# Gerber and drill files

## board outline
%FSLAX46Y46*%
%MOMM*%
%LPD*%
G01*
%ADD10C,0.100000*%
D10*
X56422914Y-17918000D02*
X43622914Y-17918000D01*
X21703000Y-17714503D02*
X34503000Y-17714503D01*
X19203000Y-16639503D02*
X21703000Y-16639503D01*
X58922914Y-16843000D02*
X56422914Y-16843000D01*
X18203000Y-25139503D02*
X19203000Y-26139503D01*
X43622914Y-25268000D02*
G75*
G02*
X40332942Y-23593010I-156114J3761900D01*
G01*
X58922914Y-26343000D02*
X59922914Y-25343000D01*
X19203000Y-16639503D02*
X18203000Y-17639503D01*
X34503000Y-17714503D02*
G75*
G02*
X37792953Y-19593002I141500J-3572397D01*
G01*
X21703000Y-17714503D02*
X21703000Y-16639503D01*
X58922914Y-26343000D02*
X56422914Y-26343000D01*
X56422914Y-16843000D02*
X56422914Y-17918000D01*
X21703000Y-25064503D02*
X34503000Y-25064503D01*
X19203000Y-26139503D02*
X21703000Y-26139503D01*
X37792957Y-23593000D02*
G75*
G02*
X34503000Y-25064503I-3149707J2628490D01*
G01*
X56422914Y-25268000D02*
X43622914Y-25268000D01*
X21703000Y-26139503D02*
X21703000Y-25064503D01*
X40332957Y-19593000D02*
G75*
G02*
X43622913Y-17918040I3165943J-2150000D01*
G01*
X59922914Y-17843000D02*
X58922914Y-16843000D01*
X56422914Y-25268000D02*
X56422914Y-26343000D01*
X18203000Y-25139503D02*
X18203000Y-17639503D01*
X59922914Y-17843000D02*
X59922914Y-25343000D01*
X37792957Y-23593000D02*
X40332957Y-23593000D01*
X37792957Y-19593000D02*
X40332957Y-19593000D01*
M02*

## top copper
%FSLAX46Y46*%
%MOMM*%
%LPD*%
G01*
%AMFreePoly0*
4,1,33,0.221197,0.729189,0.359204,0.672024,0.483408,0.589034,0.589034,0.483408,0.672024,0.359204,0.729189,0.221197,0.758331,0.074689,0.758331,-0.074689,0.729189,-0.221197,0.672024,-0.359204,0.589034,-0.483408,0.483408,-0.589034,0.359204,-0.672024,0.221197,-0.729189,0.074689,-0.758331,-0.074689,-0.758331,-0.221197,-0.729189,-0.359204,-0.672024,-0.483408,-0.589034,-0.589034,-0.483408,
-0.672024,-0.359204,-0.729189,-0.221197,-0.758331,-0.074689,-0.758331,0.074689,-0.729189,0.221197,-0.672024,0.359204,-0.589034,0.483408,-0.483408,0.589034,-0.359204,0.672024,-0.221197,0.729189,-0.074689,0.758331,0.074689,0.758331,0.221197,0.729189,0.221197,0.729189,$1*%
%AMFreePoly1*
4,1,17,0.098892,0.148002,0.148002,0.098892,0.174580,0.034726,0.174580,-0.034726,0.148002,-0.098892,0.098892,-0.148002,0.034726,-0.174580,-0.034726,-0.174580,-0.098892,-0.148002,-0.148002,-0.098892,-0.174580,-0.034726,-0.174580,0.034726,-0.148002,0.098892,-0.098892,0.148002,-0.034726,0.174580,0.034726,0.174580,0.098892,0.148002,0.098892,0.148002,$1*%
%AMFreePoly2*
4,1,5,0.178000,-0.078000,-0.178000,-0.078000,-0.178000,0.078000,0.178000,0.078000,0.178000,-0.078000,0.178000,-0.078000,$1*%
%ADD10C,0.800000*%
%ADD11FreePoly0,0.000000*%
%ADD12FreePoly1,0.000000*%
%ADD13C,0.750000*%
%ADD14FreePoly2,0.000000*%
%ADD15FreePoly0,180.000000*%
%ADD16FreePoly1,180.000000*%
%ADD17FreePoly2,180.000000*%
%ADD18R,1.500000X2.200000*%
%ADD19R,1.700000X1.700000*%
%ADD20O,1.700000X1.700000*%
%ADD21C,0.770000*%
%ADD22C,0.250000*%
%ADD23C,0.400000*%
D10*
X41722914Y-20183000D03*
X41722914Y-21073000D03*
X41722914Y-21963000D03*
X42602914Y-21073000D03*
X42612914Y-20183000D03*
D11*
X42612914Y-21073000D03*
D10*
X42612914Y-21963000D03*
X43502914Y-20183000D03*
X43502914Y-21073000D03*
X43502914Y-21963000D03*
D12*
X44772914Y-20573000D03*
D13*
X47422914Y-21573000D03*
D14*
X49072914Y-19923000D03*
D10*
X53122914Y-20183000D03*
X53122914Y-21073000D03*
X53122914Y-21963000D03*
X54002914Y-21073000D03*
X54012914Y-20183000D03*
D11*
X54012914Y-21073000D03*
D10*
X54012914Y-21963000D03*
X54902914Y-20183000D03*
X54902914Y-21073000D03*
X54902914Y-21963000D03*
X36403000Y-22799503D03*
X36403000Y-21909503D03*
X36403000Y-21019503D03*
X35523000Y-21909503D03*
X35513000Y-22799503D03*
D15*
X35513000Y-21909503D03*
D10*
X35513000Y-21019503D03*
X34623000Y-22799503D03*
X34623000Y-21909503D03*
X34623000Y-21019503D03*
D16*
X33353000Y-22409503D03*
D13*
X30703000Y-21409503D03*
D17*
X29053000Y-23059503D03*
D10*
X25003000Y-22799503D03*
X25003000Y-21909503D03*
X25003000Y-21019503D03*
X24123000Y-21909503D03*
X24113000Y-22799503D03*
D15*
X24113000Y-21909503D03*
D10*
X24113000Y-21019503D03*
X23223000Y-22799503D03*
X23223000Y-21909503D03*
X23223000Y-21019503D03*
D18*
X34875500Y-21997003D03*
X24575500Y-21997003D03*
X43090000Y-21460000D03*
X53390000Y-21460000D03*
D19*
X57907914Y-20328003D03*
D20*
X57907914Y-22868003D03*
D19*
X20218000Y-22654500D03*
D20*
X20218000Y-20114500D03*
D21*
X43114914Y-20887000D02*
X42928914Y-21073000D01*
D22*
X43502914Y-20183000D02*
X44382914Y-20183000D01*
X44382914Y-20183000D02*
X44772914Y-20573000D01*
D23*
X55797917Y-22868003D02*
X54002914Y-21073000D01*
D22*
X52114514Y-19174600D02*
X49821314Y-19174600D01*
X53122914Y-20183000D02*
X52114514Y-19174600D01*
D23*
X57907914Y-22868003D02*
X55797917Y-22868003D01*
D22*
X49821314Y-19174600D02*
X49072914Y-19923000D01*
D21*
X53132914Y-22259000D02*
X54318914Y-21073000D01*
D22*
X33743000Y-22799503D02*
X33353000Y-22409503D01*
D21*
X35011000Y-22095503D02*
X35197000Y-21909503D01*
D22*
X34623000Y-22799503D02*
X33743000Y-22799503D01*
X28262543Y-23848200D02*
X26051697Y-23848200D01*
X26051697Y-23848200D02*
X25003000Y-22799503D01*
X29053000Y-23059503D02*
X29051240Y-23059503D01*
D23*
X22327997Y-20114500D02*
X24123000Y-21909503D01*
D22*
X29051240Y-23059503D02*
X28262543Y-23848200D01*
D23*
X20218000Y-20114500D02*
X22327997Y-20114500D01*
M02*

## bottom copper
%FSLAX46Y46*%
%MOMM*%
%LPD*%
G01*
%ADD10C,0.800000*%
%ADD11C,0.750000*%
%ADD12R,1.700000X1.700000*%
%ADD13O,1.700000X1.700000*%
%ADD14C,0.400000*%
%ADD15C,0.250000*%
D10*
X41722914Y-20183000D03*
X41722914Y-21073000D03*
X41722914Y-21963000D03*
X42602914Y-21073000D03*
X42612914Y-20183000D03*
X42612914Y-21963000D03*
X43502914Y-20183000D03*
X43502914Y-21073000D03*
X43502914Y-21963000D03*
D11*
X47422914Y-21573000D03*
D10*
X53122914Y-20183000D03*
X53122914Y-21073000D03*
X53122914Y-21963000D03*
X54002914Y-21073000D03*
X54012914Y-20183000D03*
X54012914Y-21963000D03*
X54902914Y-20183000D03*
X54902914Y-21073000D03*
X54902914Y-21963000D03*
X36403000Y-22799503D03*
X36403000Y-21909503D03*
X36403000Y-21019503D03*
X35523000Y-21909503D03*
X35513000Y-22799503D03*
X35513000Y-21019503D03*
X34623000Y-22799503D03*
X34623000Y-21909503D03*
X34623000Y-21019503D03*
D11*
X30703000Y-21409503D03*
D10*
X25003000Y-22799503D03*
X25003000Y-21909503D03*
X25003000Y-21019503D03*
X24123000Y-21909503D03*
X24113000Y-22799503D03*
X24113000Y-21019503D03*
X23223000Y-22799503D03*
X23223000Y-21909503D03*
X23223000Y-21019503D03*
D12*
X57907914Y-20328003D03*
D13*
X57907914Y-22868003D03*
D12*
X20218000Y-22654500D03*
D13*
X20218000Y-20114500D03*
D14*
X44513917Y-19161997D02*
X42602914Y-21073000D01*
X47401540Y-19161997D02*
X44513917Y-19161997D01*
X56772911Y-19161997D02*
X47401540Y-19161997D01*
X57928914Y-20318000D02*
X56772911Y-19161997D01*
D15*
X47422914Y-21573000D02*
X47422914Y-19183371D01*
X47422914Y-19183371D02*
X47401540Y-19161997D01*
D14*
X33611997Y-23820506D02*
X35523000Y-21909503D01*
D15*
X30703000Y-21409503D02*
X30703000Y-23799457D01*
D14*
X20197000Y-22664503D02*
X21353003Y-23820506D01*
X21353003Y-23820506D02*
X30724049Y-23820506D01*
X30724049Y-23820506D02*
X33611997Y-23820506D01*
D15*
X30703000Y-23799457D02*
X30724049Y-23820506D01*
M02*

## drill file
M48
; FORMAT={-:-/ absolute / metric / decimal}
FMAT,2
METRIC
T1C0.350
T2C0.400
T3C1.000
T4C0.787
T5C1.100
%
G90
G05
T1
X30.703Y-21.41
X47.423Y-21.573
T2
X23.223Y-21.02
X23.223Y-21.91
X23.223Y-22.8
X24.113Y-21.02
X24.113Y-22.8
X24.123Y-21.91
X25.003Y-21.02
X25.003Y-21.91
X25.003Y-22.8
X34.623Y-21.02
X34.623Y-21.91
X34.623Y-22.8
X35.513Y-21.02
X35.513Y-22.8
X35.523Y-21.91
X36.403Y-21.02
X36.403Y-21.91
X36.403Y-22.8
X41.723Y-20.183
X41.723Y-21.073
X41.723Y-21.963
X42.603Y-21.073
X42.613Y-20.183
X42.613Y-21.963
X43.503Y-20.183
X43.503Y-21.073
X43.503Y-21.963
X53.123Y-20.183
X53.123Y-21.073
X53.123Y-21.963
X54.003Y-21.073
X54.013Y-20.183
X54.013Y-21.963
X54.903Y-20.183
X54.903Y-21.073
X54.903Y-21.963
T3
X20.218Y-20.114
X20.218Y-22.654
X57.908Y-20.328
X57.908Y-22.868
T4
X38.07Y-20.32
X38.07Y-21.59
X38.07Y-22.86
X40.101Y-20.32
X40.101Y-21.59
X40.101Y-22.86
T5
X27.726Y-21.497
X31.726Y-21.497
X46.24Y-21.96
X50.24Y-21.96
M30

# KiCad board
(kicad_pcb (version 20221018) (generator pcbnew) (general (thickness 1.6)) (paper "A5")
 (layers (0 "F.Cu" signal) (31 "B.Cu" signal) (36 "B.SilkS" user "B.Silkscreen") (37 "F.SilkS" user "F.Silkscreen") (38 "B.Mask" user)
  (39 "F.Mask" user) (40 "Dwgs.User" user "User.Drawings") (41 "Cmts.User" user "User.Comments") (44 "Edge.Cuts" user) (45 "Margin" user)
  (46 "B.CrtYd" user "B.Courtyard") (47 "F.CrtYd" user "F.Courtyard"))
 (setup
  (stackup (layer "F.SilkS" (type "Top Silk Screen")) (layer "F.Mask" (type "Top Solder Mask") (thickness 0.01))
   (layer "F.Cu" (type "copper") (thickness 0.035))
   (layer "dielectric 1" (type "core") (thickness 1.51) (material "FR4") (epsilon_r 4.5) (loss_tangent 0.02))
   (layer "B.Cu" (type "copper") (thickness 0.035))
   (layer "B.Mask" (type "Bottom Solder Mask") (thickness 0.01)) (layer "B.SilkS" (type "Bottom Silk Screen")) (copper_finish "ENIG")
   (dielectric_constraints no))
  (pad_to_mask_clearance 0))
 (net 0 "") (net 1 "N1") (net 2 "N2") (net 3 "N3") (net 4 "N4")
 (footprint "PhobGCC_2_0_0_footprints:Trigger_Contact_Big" (layer "F.Cu") (at 47.422914 21.573)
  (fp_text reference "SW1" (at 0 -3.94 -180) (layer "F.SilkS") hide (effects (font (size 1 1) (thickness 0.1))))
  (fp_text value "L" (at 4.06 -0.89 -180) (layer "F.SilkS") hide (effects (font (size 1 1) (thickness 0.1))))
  (pad "1" thru_hole circle (at -5.7 -1.39) (size 0.8 0.8) (drill 0.4) (layers "*.Cu" "*.Mask") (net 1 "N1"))
  (pad "1" thru_hole circle (at -5.7 -0.5) (size 0.8 0.8) (drill 0.4) (layers "*.Cu" "*.Mask") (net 1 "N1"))
  (pad "1" thru_hole circle (at -5.7 0.39) (size 0.8 0.8) (drill 0.4) (layers "*.Cu" "*.Mask") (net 1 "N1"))
  (pad "1" thru_hole circle (at -4.82 -0.5) (size 0.8 0.8) (drill 0.4) (layers "*.Cu" "*.Mask") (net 1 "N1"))
  (pad "1" thru_hole circle (at -4.81 -1.39) (size 0.8 0.8) (drill 0.4) (layers "*.Cu" "*.Mask") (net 1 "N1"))
  (pad "1" smd custom (at -4.81 -0.5) (size 1.524 1.524) (layers "F.Cu" "F.Paste" "F.Mask") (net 1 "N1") (thermal_bridge_angle 45)
   (options (clearance outline) (anchor circle)) (primitives))
  (pad "1" thru_hole circle (at -4.81 0.39) (size 0.8 0.8) (drill 0.4) (layers "*.Cu" "*.Mask") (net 1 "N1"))
  (pad "1" thru_hole circle (at -3.92 -1.39) (size 0.8 0.8) (drill 0.4) (layers "*.Cu" "*.Mask") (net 1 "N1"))
  (pad "1" thru_hole circle (at -3.92 -0.5) (size 0.8 0.8) (drill 0.4) (layers "*.Cu" "*.Mask") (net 1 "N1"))
  (pad "1" thru_hole circle (at -3.92 0.39) (size 0.8 0.8) (drill 0.4) (layers "*.Cu" "*.Mask") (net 1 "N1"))
  (pad "1" smd custom (at -2.65 -1) (size 0.356 0.356) (layers "F.Cu" "F.Paste" "F.Mask") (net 1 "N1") (thermal_bridge_angle 45)
   (options (clearance outline) (anchor circle)) (primitives))
  (pad "1" thru_hole circle (at 0 0) (size 0.75 0.75) (drill 0.35) (layers "*.Cu" "*.Mask") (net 1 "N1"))
  (pad "2" smd custom (at 1.65 -1.65) (size 0.356 0.156) (layers "F.Cu" "F.Paste" "F.Mask") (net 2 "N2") (thermal_bridge_angle 45)
   (options (clearance outline) (anchor rect)) (primitives))
  (pad "2" thru_hole circle (at 5.7 -1.39) (size 0.8 0.8) (drill 0.4) (layers "*.Cu" "*.Mask") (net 2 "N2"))
  (pad "2" thru_hole circle (at 5.7 -0.5) (size 0.8 0.8) (drill 0.4) (layers "*.Cu" "*.Mask") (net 2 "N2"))
  (pad "2" thru_hole circle (at 5.7 0.39) (size 0.8 0.8) (drill 0.4) (layers "*.Cu" "*.Mask") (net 2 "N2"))
  (pad "2" thru_hole circle (at 6.58 -0.5) (size 0.8 0.8) (drill 0.4) (layers "*.Cu" "*.Mask") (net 2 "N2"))
  (pad "2" thru_hole circle (at 6.59 -1.39) (size 0.8 0.8) (drill 0.4) (layers "*.Cu" "*.Mask") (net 2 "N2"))
  (pad "2" smd custom (at 6.59 -0.5) (size 1.524 1.524) (layers "F.Cu" "F.Paste" "F.Mask") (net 2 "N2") (thermal_bridge_angle 45)
   (options (clearance outline) (anchor circle)) (primitives))
  (pad "2" thru_hole circle (at 6.59 0.39) (size 0.8 0.8) (drill 0.4) (layers "*.Cu" "*.Mask") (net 2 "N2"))
  (pad "2" thru_hole circle (at 7.48 -1.39) (size 0.8 0.8) (drill 0.4) (layers "*.Cu" "*.Mask") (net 2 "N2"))
  (pad "2" thru_hole circle (at 7.48 -0.5) (size 0.8 0.8) (drill 0.4) (layers "*.Cu" "*.Mask") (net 2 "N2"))
  (pad "2" thru_hole circle (at 7.48 0.39) (size 0.8 0.8) (drill 0.4) (layers "*.Cu" "*.Mask") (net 2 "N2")))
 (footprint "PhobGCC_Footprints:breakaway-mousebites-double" (layer "F.Cu") (at 40.33085 21.36 90)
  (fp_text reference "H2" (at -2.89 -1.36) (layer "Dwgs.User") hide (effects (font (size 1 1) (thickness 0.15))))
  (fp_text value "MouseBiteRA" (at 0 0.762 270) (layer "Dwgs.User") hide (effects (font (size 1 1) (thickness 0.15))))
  (fp_line (start -2.233 -2.537893) (end -2.233 0.002107) (stroke (width 0.1) (type solid)) (layer "Edge.Cuts"))
  (fp_line (start 1.767 -2.537893) (end 1.767 0.002107) (stroke (width 0.1) (type solid)) (layer "Edge.Cuts"))
  (pad "" np_thru_hole circle (at -1.5 -2.26085 270) (size 0.7874 0.7874) (drill 0.7874) (layers "*.Cu" "*.Mask"))
  (pad "" np_thru_hole circle (at -1.5 -0.23 90) (size 0.7874 0.7874) (drill 0.7874) (layers "*.Cu" "*.Mask"))
  (pad "" np_thru_hole circle (at -0.23 -2.26085 270) (size 0.7874 0.7874) (drill 0.7874) (layers "*.Cu" "*.Mask"))
  (pad "" np_thru_hole circle (at -0.23 -0.23 90) (size 0.7874 0.7874) (drill 0.7874) (layers "*.Cu" "*.Mask"))
  (pad "" np_thru_hole circle (at 1.04 -2.26085 270) (size 0.7874 0.7874) (drill 0.7874) (layers "*.Cu" "*.Mask"))
  (pad "" np_thru_hole circle (at 1.04 -0.23 90) (size 0.7874 0.7874) (drill 0.7874) (layers "*.Cu" "*.Mask")))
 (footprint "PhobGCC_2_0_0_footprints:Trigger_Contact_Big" (layer "F.Cu") (at 30.703 21.409503 180)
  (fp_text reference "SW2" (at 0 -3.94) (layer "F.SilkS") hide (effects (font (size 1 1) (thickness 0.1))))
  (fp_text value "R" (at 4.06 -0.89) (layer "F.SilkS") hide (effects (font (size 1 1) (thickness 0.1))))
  (pad "1" thru_hole circle (at -5.7 -1.39 180) (size 0.8 0.8) (drill 0.4) (layers "*.Cu" "*.Mask") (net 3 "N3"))
  (pad "1" thru_hole circle (at -5.7 -0.5 180) (size 0.8 0.8) (drill 0.4) (layers "*.Cu" "*.Mask") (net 3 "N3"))
  (pad "1" thru_hole circle (at -5.7 0.39 180) (size 0.8 0.8) (drill 0.4) (layers "*.Cu" "*.Mask") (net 3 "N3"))
  (pad "1" thru_hole circle (at -4.82 -0.5 180) (size 0.8 0.8) (drill 0.4) (layers "*.Cu" "*.Mask") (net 3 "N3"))
  (pad "1" thru_hole circle (at -4.81 -1.39 180) (size 0.8 0.8) (drill 0.4) (layers "*.Cu" "*.Mask") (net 3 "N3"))
  (pad "1" smd custom (at -4.81 -0.5 180) (size 1.524 1.524) (layers "F.Cu" "F.Paste" "F.Mask") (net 3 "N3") (thermal_bridge_angle 45)
   (options (clearance outline) (anchor circle)) (primitives))
  (pad "1" thru_hole circle (at -4.81 0.39 180) (size 0.8 0.8) (drill 0.4) (layers "*.Cu" "*.Mask") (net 3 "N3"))
  (pad "1" thru_hole circle (at -3.92 -1.39 180) (size 0.8 0.8) (drill 0.4) (layers "*.Cu" "*.Mask") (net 3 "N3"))
  (pad "1" thru_hole circle (at -3.92 -0.5 180) (size 0.8 0.8) (drill 0.4) (layers "*.Cu" "*.Mask") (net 3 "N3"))
  (pad "1" thru_hole circle (at -3.92 0.39 180) (size 0.8 0.8) (drill 0.4) (layers "*.Cu" "*.Mask") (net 3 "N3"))
  (pad "1" smd custom (at -2.65 -1 180) (size 0.356 0.356) (layers "F.Cu" "F.Paste" "F.Mask") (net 3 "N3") (thermal_bridge_angle 45)
   (options (clearance outline) (anchor circle)) (primitives))
  (pad "1" thru_hole circle (at 0 0 180) (size 0.75 0.75) (drill 0.35) (layers "*.Cu" "*.Mask") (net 3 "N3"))
  (pad "2" smd custom (at 1.65 -1.65 180) (size 0.356 0.156) (layers "F.Cu" "F.Paste" "F.Mask") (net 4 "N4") (thermal_bridge_angle 45)
   (options (clearance outline) (anchor rect)) (primitives))
  (pad "2" thru_hole circle (at 5.7 -1.39 180) (size 0.8 0.8) (drill 0.4) (layers "*.Cu" "*.Mask") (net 4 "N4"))
  (pad "2" thru_hole circle (at 5.7 -0.5 180) (size 0.8 0.8) (drill 0.4) (layers "*.Cu" "*.Mask") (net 4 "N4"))
  (pad "2" thru_hole circle (at 5.7 0.39 180) (size 0.8 0.8) (drill 0.4) (layers "*.Cu" "*.Mask") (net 4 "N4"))
  (pad "2" thru_hole circle (at 6.58 -0.5 180) (size 0.8 0.8) (drill 0.4) (layers "*.Cu" "*.Mask") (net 4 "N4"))
  (pad "2" thru_hole circle (at 6.59 -1.39 180) (size 0.8 0.8) (drill 0.4) (layers "*.Cu" "*.Mask") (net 4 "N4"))
  (pad "2" smd custom (at 6.59 -0.5 180) (size 1.524 1.524) (layers "F.Cu" "F.Paste" "F.Mask") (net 4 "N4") (thermal_bridge_angle 45)
   (options (clearance outline) (anchor circle)) (primitives))
  (pad "2" thru_hole circle (at 6.59 0.39 180) (size 0.8 0.8) (drill 0.4) (layers "*.Cu" "*.Mask") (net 4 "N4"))
  (pad "2" thru_hole circle (at 7.48 -1.39 180) (size 0.8 0.8) (drill 0.4) (layers "*.Cu" "*.Mask") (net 4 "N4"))
  (pad "2" thru_hole circle (at 7.48 -0.5 180) (size 0.8 0.8) (drill 0.4) (layers "*.Cu" "*.Mask") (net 4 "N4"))
  (pad "2" thru_hole circle (at 7.48 0.39 180) (size 0.8 0.8) (drill 0.4) (layers "*.Cu" "*.Mask") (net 4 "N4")))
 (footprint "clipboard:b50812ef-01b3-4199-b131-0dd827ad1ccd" (layer "F.Cu") (at 35.6505 18.997003 180)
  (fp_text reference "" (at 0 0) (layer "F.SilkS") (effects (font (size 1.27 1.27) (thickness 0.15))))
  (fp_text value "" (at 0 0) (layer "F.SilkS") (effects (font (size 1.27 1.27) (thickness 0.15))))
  (pad "" np_thru_hole circle (at 3.925 -2.5 180) (size 1.1 1.1) (drill 1.1) (layers "*.Cu" "*.Mask"))
  (pad "" np_thru_hole circle (at 7.925 -2.5 180) (size 1.1 1.1) (drill 1.1) (layers "*.Cu" "*.Mask"))
  (pad "1" smd rect (at 0.775 -3 180) (size 1.5 2.2) (layers "F.Cu" "F.Mask"))
  (pad "2" smd rect (at 11.075 -3 180) (size 1.5 2.2) (layers "F.Cu" "F.Mask")))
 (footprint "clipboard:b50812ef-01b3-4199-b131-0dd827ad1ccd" (layer "F.Cu") (at 42.315 24.46)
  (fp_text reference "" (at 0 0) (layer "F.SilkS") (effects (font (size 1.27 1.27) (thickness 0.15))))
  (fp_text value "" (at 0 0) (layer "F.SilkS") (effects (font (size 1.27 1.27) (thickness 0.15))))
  (pad "" np_thru_hole circle (at 3.925 -2.5) (size 1.1 1.1) (drill 1.1) (layers "*.Cu" "*.Mask"))
  (pad "" np_thru_hole circle (at 7.925 -2.5) (size 1.1 1.1) (drill 1.1) (layers "*.Cu" "*.Mask"))
  (pad "1" smd rect (at 0.775 -3) (size 1.5 2.2) (layers "F.Cu" "F.Mask"))
  (pad "2" smd rect (at 11.075 -3) (size 1.5 2.2) (layers "F.Cu" "F.Mask")))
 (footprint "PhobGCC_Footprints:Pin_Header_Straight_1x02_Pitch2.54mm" (layer "B.Cu") (at 57.907914 20.328003 180)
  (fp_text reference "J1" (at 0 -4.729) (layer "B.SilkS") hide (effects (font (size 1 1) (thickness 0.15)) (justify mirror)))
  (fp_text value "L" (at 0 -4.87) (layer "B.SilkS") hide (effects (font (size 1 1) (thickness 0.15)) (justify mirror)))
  (pad "1" thru_hole rect (at 0 0 180) (size 1.7 1.7) (drill 1) (layers "*.Cu" "*.Mask") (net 1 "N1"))
  (pad "2" thru_hole oval (at 0 -2.54 180) (size 1.7 1.7) (drill 1) (layers "*.Cu" "*.Mask") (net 2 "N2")))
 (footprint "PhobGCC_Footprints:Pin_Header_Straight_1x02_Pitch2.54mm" (layer "B.Cu") (at 20.218 22.6545)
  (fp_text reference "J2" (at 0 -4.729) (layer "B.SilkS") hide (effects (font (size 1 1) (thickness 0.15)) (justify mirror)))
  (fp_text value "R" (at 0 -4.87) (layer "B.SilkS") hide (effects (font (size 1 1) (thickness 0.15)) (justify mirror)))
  (pad "1" thru_hole rect (at 0 0) (size 1.7 1.7) (drill 1) (layers "*.Cu" "*.Mask") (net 3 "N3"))
  (pad "2" thru_hole oval (at 0 -2.54) (size 1.7 1.7) (drill 1) (layers "*.Cu" "*.Mask") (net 4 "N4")))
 (gr_line (start 56.422914 17.918) (end 43.622914 17.918) (stroke (width 0.1) (type solid)) (layer "Edge.Cuts"))
 (gr_line (start 21.703 17.714503) (end 34.503 17.714503) (stroke (width 0.1) (type solid)) (layer "Edge.Cuts"))
 (gr_line (start 19.203 16.639503) (end 21.703 16.639503) (stroke (width 0.1) (type solid)) (layer "Edge.Cuts"))
 (gr_line (start 58.922914 16.843) (end 56.422914 16.843) (stroke (width 0.1) (type solid)) (layer "Edge.Cuts"))
 (gr_line (start 18.203 25.139503) (end 19.203 26.139503) (stroke (width 0.1) (type solid)) (layer "Edge.Cuts"))
 (gr_arc (start 43.622914 25.268) (mid 41.758548 24.861403) (end 40.332957 23.593) (stroke (width 0.1) (type solid)) (layer "Edge.Cuts"))
 (gr_line (start 58.922914 26.343) (end 59.922914 25.343) (stroke (width 0.1) (type solid)) (layer "Edge.Cuts"))
 (gr_line (start 19.203 16.639503) (end 18.203 17.639503) (stroke (width 0.1) (type solid)) (layer "Edge.Cuts"))
 (gr_arc (start 34.503 17.714503) (mid 36.41725 18.18215) (end 37.792957 19.593) (stroke (width 0.1) (type solid)) (layer "Edge.Cuts"))
 (gr_line (start 21.703 17.714503) (end 21.703 16.639503) (stroke (width 0.1) (type solid)) (layer "Edge.Cuts"))
 (gr_line (start 58.922914 26.343) (end 56.422914 26.343) (stroke (width 0.1) (type solid)) (layer "Edge.Cuts"))
 (gr_line (start 56.422914 16.843) (end 56.422914 17.918) (stroke (width 0.1) (type solid)) (layer "Edge.Cuts"))
 (gr_line (start 21.703 25.064503) (end 34.503 25.064503) (stroke (width 0.1) (type solid)) (layer "Edge.Cuts"))
 (gr_line (start 19.203 26.139503) (end 21.703 26.139503) (stroke (width 0.1) (type solid)) (layer "Edge.Cuts"))
 (gr_arc (start 37.792957 23.593) (mid 36.318224 24.709383) (end 34.503 25.064503) (stroke (width 0.1) (type solid)) (layer "Edge.Cuts"))
 (gr_line (start 56.422914 25.268) (end 43.622914 25.268) (stroke (width 0.1) (type solid)) (layer "Edge.Cuts"))
 (gr_line (start 21.703 26.139503) (end 21.703 25.064503) (stroke (width 0.1) (type solid)) (layer "Edge.Cuts"))
 (gr_arc (start 40.332957 19.593) (mid 41.762608 18.332554) (end 43.622914 17.918) (stroke (width 0.1) (type solid)) (layer "Edge.Cuts"))
 (gr_line (start 59.922914 17.843) (end 58.922914 16.843) (stroke (width 0.1) (type solid)) (layer "Edge.Cuts"))
 (gr_line (start 56.422914 25.268) (end 56.422914 26.343) (stroke (width 0.1) (type solid)) (layer "Edge.Cuts"))
 (gr_line (start 18.203 25.139503) (end 18.203 17.639503) (stroke (width 0.1) (type solid)) (layer "Edge.Cuts"))
 (gr_line (start 59.922914 17.843) (end 59.922914 25.343) (stroke (width 0.1) (type solid)) (layer "Edge.Cuts"))
 (segment (start 43.114914 20.887) (end 42.928914 21.073) (width 0.77) (layer "F.Cu") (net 1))
 (segment (start 43.502914 20.183) (end 44.382914 20.183) (width 0.25) (layer "F.Cu") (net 1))
 (segment (start 44.382914 20.183) (end 44.772914 20.573) (width 0.25) (layer "F.Cu") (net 1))
 (segment (start 44.513917 19.161997) (end 42.602914 21.073) (width 0.4) (layer "B.Cu") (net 1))
 (segment (start 47.40154 19.161997) (end 44.513917 19.161997) (width 0.4) (layer "B.Cu") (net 1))
 (segment (start 56.772911 19.161997) (end 47.40154 19.161997) (width 0.4) (layer "B.Cu") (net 1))
 (segment (start 57.928914 20.318) (end 56.772911 19.161997) (width 0.4) (layer "B.Cu") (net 1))
 (segment (start 47.422914 21.573) (end 47.422914 19.183371) (width 0.25) (layer "B.Cu") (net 1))
 (segment (start 47.422914 19.183371) (end 47.40154 19.161997) (width 0.25) (layer "B.Cu") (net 1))
 (segment (start 55.797917 22.868003) (end 54.002914 21.073) (width 0.4) (layer "F.Cu") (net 2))
 (segment (start 52.114514 19.1746) (end 49.821314 19.1746) (width 0.25) (layer "F.Cu") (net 2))
 (segment (start 53.122914 20.183) (end 52.114514 19.1746) (width 0.25) (layer "F.Cu") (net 2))
 (segment (start 57.907914 22.868003) (end 55.797917 22.868003) (width 0.4) (layer "F.Cu") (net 2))
 (segment (start 49.821314 19.1746) (end 49.072914 19.923) (width 0.25) (layer "F.Cu") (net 2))
 (segment (start 53.132914 22.259) (end 54.318914 21.073) (width 0.77) (layer "F.Cu") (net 2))
 (segment (start 33.743 22.799503) (end 33.353 22.409503) (width 0.25) (layer "F.Cu") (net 3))
 (segment (start 35.011 22.095503) (end 35.197 21.909503) (width 0.77) (layer "F.Cu") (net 3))
 (segment (start 34.623 22.799503) (end 33.743 22.799503) (width 0.25) (layer "F.Cu") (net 3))
 (segment (start 33.611997 23.820506) (end 35.523 21.909503) (width 0.4) (layer "B.Cu") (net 3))
 (segment (start 30.703 21.409503) (end 30.703 23.799457) (width 0.25) (layer "B.Cu") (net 3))
 (segment (start 20.197 22.664503) (end 21.353003 23.820506) (width 0.4) (layer "B.Cu") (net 3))
 (segment (start 21.353003 23.820506) (end 30.724049 23.820506) (width 0.4) (layer "B.Cu") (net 3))
 (segment (start 30.724049 23.820506) (end 33.611997 23.820506) (width 0.4) (layer "B.Cu") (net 3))
 (segment (start 30.703 23.799457) (end 30.724049 23.820506) (width 0.25) (layer "B.Cu") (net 3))
 (segment (start 28.262543 23.8482) (end 26.051697 23.8482) (width 0.25) (layer "F.Cu") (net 4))
 (segment (start 26.051697 23.8482) (end 25.003 22.799503) (width 0.25) (layer "F.Cu") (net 4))
 (segment (start 29.053 23.059503) (end 29.05124 23.059503) (width 0.25) (layer "F.Cu") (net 4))
 (segment (start 22.327997 20.1145) (end 24.123 21.909503) (width 0.4) (layer "F.Cu") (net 4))
 (segment (start 29.05124 23.059503) (end 28.262543 23.8482) (width 0.25) (layer "F.Cu") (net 4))
 (segment (start 20.218 20.1145) (end 22.327997 20.1145) (width 0.4) (layer "F.Cu") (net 4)))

